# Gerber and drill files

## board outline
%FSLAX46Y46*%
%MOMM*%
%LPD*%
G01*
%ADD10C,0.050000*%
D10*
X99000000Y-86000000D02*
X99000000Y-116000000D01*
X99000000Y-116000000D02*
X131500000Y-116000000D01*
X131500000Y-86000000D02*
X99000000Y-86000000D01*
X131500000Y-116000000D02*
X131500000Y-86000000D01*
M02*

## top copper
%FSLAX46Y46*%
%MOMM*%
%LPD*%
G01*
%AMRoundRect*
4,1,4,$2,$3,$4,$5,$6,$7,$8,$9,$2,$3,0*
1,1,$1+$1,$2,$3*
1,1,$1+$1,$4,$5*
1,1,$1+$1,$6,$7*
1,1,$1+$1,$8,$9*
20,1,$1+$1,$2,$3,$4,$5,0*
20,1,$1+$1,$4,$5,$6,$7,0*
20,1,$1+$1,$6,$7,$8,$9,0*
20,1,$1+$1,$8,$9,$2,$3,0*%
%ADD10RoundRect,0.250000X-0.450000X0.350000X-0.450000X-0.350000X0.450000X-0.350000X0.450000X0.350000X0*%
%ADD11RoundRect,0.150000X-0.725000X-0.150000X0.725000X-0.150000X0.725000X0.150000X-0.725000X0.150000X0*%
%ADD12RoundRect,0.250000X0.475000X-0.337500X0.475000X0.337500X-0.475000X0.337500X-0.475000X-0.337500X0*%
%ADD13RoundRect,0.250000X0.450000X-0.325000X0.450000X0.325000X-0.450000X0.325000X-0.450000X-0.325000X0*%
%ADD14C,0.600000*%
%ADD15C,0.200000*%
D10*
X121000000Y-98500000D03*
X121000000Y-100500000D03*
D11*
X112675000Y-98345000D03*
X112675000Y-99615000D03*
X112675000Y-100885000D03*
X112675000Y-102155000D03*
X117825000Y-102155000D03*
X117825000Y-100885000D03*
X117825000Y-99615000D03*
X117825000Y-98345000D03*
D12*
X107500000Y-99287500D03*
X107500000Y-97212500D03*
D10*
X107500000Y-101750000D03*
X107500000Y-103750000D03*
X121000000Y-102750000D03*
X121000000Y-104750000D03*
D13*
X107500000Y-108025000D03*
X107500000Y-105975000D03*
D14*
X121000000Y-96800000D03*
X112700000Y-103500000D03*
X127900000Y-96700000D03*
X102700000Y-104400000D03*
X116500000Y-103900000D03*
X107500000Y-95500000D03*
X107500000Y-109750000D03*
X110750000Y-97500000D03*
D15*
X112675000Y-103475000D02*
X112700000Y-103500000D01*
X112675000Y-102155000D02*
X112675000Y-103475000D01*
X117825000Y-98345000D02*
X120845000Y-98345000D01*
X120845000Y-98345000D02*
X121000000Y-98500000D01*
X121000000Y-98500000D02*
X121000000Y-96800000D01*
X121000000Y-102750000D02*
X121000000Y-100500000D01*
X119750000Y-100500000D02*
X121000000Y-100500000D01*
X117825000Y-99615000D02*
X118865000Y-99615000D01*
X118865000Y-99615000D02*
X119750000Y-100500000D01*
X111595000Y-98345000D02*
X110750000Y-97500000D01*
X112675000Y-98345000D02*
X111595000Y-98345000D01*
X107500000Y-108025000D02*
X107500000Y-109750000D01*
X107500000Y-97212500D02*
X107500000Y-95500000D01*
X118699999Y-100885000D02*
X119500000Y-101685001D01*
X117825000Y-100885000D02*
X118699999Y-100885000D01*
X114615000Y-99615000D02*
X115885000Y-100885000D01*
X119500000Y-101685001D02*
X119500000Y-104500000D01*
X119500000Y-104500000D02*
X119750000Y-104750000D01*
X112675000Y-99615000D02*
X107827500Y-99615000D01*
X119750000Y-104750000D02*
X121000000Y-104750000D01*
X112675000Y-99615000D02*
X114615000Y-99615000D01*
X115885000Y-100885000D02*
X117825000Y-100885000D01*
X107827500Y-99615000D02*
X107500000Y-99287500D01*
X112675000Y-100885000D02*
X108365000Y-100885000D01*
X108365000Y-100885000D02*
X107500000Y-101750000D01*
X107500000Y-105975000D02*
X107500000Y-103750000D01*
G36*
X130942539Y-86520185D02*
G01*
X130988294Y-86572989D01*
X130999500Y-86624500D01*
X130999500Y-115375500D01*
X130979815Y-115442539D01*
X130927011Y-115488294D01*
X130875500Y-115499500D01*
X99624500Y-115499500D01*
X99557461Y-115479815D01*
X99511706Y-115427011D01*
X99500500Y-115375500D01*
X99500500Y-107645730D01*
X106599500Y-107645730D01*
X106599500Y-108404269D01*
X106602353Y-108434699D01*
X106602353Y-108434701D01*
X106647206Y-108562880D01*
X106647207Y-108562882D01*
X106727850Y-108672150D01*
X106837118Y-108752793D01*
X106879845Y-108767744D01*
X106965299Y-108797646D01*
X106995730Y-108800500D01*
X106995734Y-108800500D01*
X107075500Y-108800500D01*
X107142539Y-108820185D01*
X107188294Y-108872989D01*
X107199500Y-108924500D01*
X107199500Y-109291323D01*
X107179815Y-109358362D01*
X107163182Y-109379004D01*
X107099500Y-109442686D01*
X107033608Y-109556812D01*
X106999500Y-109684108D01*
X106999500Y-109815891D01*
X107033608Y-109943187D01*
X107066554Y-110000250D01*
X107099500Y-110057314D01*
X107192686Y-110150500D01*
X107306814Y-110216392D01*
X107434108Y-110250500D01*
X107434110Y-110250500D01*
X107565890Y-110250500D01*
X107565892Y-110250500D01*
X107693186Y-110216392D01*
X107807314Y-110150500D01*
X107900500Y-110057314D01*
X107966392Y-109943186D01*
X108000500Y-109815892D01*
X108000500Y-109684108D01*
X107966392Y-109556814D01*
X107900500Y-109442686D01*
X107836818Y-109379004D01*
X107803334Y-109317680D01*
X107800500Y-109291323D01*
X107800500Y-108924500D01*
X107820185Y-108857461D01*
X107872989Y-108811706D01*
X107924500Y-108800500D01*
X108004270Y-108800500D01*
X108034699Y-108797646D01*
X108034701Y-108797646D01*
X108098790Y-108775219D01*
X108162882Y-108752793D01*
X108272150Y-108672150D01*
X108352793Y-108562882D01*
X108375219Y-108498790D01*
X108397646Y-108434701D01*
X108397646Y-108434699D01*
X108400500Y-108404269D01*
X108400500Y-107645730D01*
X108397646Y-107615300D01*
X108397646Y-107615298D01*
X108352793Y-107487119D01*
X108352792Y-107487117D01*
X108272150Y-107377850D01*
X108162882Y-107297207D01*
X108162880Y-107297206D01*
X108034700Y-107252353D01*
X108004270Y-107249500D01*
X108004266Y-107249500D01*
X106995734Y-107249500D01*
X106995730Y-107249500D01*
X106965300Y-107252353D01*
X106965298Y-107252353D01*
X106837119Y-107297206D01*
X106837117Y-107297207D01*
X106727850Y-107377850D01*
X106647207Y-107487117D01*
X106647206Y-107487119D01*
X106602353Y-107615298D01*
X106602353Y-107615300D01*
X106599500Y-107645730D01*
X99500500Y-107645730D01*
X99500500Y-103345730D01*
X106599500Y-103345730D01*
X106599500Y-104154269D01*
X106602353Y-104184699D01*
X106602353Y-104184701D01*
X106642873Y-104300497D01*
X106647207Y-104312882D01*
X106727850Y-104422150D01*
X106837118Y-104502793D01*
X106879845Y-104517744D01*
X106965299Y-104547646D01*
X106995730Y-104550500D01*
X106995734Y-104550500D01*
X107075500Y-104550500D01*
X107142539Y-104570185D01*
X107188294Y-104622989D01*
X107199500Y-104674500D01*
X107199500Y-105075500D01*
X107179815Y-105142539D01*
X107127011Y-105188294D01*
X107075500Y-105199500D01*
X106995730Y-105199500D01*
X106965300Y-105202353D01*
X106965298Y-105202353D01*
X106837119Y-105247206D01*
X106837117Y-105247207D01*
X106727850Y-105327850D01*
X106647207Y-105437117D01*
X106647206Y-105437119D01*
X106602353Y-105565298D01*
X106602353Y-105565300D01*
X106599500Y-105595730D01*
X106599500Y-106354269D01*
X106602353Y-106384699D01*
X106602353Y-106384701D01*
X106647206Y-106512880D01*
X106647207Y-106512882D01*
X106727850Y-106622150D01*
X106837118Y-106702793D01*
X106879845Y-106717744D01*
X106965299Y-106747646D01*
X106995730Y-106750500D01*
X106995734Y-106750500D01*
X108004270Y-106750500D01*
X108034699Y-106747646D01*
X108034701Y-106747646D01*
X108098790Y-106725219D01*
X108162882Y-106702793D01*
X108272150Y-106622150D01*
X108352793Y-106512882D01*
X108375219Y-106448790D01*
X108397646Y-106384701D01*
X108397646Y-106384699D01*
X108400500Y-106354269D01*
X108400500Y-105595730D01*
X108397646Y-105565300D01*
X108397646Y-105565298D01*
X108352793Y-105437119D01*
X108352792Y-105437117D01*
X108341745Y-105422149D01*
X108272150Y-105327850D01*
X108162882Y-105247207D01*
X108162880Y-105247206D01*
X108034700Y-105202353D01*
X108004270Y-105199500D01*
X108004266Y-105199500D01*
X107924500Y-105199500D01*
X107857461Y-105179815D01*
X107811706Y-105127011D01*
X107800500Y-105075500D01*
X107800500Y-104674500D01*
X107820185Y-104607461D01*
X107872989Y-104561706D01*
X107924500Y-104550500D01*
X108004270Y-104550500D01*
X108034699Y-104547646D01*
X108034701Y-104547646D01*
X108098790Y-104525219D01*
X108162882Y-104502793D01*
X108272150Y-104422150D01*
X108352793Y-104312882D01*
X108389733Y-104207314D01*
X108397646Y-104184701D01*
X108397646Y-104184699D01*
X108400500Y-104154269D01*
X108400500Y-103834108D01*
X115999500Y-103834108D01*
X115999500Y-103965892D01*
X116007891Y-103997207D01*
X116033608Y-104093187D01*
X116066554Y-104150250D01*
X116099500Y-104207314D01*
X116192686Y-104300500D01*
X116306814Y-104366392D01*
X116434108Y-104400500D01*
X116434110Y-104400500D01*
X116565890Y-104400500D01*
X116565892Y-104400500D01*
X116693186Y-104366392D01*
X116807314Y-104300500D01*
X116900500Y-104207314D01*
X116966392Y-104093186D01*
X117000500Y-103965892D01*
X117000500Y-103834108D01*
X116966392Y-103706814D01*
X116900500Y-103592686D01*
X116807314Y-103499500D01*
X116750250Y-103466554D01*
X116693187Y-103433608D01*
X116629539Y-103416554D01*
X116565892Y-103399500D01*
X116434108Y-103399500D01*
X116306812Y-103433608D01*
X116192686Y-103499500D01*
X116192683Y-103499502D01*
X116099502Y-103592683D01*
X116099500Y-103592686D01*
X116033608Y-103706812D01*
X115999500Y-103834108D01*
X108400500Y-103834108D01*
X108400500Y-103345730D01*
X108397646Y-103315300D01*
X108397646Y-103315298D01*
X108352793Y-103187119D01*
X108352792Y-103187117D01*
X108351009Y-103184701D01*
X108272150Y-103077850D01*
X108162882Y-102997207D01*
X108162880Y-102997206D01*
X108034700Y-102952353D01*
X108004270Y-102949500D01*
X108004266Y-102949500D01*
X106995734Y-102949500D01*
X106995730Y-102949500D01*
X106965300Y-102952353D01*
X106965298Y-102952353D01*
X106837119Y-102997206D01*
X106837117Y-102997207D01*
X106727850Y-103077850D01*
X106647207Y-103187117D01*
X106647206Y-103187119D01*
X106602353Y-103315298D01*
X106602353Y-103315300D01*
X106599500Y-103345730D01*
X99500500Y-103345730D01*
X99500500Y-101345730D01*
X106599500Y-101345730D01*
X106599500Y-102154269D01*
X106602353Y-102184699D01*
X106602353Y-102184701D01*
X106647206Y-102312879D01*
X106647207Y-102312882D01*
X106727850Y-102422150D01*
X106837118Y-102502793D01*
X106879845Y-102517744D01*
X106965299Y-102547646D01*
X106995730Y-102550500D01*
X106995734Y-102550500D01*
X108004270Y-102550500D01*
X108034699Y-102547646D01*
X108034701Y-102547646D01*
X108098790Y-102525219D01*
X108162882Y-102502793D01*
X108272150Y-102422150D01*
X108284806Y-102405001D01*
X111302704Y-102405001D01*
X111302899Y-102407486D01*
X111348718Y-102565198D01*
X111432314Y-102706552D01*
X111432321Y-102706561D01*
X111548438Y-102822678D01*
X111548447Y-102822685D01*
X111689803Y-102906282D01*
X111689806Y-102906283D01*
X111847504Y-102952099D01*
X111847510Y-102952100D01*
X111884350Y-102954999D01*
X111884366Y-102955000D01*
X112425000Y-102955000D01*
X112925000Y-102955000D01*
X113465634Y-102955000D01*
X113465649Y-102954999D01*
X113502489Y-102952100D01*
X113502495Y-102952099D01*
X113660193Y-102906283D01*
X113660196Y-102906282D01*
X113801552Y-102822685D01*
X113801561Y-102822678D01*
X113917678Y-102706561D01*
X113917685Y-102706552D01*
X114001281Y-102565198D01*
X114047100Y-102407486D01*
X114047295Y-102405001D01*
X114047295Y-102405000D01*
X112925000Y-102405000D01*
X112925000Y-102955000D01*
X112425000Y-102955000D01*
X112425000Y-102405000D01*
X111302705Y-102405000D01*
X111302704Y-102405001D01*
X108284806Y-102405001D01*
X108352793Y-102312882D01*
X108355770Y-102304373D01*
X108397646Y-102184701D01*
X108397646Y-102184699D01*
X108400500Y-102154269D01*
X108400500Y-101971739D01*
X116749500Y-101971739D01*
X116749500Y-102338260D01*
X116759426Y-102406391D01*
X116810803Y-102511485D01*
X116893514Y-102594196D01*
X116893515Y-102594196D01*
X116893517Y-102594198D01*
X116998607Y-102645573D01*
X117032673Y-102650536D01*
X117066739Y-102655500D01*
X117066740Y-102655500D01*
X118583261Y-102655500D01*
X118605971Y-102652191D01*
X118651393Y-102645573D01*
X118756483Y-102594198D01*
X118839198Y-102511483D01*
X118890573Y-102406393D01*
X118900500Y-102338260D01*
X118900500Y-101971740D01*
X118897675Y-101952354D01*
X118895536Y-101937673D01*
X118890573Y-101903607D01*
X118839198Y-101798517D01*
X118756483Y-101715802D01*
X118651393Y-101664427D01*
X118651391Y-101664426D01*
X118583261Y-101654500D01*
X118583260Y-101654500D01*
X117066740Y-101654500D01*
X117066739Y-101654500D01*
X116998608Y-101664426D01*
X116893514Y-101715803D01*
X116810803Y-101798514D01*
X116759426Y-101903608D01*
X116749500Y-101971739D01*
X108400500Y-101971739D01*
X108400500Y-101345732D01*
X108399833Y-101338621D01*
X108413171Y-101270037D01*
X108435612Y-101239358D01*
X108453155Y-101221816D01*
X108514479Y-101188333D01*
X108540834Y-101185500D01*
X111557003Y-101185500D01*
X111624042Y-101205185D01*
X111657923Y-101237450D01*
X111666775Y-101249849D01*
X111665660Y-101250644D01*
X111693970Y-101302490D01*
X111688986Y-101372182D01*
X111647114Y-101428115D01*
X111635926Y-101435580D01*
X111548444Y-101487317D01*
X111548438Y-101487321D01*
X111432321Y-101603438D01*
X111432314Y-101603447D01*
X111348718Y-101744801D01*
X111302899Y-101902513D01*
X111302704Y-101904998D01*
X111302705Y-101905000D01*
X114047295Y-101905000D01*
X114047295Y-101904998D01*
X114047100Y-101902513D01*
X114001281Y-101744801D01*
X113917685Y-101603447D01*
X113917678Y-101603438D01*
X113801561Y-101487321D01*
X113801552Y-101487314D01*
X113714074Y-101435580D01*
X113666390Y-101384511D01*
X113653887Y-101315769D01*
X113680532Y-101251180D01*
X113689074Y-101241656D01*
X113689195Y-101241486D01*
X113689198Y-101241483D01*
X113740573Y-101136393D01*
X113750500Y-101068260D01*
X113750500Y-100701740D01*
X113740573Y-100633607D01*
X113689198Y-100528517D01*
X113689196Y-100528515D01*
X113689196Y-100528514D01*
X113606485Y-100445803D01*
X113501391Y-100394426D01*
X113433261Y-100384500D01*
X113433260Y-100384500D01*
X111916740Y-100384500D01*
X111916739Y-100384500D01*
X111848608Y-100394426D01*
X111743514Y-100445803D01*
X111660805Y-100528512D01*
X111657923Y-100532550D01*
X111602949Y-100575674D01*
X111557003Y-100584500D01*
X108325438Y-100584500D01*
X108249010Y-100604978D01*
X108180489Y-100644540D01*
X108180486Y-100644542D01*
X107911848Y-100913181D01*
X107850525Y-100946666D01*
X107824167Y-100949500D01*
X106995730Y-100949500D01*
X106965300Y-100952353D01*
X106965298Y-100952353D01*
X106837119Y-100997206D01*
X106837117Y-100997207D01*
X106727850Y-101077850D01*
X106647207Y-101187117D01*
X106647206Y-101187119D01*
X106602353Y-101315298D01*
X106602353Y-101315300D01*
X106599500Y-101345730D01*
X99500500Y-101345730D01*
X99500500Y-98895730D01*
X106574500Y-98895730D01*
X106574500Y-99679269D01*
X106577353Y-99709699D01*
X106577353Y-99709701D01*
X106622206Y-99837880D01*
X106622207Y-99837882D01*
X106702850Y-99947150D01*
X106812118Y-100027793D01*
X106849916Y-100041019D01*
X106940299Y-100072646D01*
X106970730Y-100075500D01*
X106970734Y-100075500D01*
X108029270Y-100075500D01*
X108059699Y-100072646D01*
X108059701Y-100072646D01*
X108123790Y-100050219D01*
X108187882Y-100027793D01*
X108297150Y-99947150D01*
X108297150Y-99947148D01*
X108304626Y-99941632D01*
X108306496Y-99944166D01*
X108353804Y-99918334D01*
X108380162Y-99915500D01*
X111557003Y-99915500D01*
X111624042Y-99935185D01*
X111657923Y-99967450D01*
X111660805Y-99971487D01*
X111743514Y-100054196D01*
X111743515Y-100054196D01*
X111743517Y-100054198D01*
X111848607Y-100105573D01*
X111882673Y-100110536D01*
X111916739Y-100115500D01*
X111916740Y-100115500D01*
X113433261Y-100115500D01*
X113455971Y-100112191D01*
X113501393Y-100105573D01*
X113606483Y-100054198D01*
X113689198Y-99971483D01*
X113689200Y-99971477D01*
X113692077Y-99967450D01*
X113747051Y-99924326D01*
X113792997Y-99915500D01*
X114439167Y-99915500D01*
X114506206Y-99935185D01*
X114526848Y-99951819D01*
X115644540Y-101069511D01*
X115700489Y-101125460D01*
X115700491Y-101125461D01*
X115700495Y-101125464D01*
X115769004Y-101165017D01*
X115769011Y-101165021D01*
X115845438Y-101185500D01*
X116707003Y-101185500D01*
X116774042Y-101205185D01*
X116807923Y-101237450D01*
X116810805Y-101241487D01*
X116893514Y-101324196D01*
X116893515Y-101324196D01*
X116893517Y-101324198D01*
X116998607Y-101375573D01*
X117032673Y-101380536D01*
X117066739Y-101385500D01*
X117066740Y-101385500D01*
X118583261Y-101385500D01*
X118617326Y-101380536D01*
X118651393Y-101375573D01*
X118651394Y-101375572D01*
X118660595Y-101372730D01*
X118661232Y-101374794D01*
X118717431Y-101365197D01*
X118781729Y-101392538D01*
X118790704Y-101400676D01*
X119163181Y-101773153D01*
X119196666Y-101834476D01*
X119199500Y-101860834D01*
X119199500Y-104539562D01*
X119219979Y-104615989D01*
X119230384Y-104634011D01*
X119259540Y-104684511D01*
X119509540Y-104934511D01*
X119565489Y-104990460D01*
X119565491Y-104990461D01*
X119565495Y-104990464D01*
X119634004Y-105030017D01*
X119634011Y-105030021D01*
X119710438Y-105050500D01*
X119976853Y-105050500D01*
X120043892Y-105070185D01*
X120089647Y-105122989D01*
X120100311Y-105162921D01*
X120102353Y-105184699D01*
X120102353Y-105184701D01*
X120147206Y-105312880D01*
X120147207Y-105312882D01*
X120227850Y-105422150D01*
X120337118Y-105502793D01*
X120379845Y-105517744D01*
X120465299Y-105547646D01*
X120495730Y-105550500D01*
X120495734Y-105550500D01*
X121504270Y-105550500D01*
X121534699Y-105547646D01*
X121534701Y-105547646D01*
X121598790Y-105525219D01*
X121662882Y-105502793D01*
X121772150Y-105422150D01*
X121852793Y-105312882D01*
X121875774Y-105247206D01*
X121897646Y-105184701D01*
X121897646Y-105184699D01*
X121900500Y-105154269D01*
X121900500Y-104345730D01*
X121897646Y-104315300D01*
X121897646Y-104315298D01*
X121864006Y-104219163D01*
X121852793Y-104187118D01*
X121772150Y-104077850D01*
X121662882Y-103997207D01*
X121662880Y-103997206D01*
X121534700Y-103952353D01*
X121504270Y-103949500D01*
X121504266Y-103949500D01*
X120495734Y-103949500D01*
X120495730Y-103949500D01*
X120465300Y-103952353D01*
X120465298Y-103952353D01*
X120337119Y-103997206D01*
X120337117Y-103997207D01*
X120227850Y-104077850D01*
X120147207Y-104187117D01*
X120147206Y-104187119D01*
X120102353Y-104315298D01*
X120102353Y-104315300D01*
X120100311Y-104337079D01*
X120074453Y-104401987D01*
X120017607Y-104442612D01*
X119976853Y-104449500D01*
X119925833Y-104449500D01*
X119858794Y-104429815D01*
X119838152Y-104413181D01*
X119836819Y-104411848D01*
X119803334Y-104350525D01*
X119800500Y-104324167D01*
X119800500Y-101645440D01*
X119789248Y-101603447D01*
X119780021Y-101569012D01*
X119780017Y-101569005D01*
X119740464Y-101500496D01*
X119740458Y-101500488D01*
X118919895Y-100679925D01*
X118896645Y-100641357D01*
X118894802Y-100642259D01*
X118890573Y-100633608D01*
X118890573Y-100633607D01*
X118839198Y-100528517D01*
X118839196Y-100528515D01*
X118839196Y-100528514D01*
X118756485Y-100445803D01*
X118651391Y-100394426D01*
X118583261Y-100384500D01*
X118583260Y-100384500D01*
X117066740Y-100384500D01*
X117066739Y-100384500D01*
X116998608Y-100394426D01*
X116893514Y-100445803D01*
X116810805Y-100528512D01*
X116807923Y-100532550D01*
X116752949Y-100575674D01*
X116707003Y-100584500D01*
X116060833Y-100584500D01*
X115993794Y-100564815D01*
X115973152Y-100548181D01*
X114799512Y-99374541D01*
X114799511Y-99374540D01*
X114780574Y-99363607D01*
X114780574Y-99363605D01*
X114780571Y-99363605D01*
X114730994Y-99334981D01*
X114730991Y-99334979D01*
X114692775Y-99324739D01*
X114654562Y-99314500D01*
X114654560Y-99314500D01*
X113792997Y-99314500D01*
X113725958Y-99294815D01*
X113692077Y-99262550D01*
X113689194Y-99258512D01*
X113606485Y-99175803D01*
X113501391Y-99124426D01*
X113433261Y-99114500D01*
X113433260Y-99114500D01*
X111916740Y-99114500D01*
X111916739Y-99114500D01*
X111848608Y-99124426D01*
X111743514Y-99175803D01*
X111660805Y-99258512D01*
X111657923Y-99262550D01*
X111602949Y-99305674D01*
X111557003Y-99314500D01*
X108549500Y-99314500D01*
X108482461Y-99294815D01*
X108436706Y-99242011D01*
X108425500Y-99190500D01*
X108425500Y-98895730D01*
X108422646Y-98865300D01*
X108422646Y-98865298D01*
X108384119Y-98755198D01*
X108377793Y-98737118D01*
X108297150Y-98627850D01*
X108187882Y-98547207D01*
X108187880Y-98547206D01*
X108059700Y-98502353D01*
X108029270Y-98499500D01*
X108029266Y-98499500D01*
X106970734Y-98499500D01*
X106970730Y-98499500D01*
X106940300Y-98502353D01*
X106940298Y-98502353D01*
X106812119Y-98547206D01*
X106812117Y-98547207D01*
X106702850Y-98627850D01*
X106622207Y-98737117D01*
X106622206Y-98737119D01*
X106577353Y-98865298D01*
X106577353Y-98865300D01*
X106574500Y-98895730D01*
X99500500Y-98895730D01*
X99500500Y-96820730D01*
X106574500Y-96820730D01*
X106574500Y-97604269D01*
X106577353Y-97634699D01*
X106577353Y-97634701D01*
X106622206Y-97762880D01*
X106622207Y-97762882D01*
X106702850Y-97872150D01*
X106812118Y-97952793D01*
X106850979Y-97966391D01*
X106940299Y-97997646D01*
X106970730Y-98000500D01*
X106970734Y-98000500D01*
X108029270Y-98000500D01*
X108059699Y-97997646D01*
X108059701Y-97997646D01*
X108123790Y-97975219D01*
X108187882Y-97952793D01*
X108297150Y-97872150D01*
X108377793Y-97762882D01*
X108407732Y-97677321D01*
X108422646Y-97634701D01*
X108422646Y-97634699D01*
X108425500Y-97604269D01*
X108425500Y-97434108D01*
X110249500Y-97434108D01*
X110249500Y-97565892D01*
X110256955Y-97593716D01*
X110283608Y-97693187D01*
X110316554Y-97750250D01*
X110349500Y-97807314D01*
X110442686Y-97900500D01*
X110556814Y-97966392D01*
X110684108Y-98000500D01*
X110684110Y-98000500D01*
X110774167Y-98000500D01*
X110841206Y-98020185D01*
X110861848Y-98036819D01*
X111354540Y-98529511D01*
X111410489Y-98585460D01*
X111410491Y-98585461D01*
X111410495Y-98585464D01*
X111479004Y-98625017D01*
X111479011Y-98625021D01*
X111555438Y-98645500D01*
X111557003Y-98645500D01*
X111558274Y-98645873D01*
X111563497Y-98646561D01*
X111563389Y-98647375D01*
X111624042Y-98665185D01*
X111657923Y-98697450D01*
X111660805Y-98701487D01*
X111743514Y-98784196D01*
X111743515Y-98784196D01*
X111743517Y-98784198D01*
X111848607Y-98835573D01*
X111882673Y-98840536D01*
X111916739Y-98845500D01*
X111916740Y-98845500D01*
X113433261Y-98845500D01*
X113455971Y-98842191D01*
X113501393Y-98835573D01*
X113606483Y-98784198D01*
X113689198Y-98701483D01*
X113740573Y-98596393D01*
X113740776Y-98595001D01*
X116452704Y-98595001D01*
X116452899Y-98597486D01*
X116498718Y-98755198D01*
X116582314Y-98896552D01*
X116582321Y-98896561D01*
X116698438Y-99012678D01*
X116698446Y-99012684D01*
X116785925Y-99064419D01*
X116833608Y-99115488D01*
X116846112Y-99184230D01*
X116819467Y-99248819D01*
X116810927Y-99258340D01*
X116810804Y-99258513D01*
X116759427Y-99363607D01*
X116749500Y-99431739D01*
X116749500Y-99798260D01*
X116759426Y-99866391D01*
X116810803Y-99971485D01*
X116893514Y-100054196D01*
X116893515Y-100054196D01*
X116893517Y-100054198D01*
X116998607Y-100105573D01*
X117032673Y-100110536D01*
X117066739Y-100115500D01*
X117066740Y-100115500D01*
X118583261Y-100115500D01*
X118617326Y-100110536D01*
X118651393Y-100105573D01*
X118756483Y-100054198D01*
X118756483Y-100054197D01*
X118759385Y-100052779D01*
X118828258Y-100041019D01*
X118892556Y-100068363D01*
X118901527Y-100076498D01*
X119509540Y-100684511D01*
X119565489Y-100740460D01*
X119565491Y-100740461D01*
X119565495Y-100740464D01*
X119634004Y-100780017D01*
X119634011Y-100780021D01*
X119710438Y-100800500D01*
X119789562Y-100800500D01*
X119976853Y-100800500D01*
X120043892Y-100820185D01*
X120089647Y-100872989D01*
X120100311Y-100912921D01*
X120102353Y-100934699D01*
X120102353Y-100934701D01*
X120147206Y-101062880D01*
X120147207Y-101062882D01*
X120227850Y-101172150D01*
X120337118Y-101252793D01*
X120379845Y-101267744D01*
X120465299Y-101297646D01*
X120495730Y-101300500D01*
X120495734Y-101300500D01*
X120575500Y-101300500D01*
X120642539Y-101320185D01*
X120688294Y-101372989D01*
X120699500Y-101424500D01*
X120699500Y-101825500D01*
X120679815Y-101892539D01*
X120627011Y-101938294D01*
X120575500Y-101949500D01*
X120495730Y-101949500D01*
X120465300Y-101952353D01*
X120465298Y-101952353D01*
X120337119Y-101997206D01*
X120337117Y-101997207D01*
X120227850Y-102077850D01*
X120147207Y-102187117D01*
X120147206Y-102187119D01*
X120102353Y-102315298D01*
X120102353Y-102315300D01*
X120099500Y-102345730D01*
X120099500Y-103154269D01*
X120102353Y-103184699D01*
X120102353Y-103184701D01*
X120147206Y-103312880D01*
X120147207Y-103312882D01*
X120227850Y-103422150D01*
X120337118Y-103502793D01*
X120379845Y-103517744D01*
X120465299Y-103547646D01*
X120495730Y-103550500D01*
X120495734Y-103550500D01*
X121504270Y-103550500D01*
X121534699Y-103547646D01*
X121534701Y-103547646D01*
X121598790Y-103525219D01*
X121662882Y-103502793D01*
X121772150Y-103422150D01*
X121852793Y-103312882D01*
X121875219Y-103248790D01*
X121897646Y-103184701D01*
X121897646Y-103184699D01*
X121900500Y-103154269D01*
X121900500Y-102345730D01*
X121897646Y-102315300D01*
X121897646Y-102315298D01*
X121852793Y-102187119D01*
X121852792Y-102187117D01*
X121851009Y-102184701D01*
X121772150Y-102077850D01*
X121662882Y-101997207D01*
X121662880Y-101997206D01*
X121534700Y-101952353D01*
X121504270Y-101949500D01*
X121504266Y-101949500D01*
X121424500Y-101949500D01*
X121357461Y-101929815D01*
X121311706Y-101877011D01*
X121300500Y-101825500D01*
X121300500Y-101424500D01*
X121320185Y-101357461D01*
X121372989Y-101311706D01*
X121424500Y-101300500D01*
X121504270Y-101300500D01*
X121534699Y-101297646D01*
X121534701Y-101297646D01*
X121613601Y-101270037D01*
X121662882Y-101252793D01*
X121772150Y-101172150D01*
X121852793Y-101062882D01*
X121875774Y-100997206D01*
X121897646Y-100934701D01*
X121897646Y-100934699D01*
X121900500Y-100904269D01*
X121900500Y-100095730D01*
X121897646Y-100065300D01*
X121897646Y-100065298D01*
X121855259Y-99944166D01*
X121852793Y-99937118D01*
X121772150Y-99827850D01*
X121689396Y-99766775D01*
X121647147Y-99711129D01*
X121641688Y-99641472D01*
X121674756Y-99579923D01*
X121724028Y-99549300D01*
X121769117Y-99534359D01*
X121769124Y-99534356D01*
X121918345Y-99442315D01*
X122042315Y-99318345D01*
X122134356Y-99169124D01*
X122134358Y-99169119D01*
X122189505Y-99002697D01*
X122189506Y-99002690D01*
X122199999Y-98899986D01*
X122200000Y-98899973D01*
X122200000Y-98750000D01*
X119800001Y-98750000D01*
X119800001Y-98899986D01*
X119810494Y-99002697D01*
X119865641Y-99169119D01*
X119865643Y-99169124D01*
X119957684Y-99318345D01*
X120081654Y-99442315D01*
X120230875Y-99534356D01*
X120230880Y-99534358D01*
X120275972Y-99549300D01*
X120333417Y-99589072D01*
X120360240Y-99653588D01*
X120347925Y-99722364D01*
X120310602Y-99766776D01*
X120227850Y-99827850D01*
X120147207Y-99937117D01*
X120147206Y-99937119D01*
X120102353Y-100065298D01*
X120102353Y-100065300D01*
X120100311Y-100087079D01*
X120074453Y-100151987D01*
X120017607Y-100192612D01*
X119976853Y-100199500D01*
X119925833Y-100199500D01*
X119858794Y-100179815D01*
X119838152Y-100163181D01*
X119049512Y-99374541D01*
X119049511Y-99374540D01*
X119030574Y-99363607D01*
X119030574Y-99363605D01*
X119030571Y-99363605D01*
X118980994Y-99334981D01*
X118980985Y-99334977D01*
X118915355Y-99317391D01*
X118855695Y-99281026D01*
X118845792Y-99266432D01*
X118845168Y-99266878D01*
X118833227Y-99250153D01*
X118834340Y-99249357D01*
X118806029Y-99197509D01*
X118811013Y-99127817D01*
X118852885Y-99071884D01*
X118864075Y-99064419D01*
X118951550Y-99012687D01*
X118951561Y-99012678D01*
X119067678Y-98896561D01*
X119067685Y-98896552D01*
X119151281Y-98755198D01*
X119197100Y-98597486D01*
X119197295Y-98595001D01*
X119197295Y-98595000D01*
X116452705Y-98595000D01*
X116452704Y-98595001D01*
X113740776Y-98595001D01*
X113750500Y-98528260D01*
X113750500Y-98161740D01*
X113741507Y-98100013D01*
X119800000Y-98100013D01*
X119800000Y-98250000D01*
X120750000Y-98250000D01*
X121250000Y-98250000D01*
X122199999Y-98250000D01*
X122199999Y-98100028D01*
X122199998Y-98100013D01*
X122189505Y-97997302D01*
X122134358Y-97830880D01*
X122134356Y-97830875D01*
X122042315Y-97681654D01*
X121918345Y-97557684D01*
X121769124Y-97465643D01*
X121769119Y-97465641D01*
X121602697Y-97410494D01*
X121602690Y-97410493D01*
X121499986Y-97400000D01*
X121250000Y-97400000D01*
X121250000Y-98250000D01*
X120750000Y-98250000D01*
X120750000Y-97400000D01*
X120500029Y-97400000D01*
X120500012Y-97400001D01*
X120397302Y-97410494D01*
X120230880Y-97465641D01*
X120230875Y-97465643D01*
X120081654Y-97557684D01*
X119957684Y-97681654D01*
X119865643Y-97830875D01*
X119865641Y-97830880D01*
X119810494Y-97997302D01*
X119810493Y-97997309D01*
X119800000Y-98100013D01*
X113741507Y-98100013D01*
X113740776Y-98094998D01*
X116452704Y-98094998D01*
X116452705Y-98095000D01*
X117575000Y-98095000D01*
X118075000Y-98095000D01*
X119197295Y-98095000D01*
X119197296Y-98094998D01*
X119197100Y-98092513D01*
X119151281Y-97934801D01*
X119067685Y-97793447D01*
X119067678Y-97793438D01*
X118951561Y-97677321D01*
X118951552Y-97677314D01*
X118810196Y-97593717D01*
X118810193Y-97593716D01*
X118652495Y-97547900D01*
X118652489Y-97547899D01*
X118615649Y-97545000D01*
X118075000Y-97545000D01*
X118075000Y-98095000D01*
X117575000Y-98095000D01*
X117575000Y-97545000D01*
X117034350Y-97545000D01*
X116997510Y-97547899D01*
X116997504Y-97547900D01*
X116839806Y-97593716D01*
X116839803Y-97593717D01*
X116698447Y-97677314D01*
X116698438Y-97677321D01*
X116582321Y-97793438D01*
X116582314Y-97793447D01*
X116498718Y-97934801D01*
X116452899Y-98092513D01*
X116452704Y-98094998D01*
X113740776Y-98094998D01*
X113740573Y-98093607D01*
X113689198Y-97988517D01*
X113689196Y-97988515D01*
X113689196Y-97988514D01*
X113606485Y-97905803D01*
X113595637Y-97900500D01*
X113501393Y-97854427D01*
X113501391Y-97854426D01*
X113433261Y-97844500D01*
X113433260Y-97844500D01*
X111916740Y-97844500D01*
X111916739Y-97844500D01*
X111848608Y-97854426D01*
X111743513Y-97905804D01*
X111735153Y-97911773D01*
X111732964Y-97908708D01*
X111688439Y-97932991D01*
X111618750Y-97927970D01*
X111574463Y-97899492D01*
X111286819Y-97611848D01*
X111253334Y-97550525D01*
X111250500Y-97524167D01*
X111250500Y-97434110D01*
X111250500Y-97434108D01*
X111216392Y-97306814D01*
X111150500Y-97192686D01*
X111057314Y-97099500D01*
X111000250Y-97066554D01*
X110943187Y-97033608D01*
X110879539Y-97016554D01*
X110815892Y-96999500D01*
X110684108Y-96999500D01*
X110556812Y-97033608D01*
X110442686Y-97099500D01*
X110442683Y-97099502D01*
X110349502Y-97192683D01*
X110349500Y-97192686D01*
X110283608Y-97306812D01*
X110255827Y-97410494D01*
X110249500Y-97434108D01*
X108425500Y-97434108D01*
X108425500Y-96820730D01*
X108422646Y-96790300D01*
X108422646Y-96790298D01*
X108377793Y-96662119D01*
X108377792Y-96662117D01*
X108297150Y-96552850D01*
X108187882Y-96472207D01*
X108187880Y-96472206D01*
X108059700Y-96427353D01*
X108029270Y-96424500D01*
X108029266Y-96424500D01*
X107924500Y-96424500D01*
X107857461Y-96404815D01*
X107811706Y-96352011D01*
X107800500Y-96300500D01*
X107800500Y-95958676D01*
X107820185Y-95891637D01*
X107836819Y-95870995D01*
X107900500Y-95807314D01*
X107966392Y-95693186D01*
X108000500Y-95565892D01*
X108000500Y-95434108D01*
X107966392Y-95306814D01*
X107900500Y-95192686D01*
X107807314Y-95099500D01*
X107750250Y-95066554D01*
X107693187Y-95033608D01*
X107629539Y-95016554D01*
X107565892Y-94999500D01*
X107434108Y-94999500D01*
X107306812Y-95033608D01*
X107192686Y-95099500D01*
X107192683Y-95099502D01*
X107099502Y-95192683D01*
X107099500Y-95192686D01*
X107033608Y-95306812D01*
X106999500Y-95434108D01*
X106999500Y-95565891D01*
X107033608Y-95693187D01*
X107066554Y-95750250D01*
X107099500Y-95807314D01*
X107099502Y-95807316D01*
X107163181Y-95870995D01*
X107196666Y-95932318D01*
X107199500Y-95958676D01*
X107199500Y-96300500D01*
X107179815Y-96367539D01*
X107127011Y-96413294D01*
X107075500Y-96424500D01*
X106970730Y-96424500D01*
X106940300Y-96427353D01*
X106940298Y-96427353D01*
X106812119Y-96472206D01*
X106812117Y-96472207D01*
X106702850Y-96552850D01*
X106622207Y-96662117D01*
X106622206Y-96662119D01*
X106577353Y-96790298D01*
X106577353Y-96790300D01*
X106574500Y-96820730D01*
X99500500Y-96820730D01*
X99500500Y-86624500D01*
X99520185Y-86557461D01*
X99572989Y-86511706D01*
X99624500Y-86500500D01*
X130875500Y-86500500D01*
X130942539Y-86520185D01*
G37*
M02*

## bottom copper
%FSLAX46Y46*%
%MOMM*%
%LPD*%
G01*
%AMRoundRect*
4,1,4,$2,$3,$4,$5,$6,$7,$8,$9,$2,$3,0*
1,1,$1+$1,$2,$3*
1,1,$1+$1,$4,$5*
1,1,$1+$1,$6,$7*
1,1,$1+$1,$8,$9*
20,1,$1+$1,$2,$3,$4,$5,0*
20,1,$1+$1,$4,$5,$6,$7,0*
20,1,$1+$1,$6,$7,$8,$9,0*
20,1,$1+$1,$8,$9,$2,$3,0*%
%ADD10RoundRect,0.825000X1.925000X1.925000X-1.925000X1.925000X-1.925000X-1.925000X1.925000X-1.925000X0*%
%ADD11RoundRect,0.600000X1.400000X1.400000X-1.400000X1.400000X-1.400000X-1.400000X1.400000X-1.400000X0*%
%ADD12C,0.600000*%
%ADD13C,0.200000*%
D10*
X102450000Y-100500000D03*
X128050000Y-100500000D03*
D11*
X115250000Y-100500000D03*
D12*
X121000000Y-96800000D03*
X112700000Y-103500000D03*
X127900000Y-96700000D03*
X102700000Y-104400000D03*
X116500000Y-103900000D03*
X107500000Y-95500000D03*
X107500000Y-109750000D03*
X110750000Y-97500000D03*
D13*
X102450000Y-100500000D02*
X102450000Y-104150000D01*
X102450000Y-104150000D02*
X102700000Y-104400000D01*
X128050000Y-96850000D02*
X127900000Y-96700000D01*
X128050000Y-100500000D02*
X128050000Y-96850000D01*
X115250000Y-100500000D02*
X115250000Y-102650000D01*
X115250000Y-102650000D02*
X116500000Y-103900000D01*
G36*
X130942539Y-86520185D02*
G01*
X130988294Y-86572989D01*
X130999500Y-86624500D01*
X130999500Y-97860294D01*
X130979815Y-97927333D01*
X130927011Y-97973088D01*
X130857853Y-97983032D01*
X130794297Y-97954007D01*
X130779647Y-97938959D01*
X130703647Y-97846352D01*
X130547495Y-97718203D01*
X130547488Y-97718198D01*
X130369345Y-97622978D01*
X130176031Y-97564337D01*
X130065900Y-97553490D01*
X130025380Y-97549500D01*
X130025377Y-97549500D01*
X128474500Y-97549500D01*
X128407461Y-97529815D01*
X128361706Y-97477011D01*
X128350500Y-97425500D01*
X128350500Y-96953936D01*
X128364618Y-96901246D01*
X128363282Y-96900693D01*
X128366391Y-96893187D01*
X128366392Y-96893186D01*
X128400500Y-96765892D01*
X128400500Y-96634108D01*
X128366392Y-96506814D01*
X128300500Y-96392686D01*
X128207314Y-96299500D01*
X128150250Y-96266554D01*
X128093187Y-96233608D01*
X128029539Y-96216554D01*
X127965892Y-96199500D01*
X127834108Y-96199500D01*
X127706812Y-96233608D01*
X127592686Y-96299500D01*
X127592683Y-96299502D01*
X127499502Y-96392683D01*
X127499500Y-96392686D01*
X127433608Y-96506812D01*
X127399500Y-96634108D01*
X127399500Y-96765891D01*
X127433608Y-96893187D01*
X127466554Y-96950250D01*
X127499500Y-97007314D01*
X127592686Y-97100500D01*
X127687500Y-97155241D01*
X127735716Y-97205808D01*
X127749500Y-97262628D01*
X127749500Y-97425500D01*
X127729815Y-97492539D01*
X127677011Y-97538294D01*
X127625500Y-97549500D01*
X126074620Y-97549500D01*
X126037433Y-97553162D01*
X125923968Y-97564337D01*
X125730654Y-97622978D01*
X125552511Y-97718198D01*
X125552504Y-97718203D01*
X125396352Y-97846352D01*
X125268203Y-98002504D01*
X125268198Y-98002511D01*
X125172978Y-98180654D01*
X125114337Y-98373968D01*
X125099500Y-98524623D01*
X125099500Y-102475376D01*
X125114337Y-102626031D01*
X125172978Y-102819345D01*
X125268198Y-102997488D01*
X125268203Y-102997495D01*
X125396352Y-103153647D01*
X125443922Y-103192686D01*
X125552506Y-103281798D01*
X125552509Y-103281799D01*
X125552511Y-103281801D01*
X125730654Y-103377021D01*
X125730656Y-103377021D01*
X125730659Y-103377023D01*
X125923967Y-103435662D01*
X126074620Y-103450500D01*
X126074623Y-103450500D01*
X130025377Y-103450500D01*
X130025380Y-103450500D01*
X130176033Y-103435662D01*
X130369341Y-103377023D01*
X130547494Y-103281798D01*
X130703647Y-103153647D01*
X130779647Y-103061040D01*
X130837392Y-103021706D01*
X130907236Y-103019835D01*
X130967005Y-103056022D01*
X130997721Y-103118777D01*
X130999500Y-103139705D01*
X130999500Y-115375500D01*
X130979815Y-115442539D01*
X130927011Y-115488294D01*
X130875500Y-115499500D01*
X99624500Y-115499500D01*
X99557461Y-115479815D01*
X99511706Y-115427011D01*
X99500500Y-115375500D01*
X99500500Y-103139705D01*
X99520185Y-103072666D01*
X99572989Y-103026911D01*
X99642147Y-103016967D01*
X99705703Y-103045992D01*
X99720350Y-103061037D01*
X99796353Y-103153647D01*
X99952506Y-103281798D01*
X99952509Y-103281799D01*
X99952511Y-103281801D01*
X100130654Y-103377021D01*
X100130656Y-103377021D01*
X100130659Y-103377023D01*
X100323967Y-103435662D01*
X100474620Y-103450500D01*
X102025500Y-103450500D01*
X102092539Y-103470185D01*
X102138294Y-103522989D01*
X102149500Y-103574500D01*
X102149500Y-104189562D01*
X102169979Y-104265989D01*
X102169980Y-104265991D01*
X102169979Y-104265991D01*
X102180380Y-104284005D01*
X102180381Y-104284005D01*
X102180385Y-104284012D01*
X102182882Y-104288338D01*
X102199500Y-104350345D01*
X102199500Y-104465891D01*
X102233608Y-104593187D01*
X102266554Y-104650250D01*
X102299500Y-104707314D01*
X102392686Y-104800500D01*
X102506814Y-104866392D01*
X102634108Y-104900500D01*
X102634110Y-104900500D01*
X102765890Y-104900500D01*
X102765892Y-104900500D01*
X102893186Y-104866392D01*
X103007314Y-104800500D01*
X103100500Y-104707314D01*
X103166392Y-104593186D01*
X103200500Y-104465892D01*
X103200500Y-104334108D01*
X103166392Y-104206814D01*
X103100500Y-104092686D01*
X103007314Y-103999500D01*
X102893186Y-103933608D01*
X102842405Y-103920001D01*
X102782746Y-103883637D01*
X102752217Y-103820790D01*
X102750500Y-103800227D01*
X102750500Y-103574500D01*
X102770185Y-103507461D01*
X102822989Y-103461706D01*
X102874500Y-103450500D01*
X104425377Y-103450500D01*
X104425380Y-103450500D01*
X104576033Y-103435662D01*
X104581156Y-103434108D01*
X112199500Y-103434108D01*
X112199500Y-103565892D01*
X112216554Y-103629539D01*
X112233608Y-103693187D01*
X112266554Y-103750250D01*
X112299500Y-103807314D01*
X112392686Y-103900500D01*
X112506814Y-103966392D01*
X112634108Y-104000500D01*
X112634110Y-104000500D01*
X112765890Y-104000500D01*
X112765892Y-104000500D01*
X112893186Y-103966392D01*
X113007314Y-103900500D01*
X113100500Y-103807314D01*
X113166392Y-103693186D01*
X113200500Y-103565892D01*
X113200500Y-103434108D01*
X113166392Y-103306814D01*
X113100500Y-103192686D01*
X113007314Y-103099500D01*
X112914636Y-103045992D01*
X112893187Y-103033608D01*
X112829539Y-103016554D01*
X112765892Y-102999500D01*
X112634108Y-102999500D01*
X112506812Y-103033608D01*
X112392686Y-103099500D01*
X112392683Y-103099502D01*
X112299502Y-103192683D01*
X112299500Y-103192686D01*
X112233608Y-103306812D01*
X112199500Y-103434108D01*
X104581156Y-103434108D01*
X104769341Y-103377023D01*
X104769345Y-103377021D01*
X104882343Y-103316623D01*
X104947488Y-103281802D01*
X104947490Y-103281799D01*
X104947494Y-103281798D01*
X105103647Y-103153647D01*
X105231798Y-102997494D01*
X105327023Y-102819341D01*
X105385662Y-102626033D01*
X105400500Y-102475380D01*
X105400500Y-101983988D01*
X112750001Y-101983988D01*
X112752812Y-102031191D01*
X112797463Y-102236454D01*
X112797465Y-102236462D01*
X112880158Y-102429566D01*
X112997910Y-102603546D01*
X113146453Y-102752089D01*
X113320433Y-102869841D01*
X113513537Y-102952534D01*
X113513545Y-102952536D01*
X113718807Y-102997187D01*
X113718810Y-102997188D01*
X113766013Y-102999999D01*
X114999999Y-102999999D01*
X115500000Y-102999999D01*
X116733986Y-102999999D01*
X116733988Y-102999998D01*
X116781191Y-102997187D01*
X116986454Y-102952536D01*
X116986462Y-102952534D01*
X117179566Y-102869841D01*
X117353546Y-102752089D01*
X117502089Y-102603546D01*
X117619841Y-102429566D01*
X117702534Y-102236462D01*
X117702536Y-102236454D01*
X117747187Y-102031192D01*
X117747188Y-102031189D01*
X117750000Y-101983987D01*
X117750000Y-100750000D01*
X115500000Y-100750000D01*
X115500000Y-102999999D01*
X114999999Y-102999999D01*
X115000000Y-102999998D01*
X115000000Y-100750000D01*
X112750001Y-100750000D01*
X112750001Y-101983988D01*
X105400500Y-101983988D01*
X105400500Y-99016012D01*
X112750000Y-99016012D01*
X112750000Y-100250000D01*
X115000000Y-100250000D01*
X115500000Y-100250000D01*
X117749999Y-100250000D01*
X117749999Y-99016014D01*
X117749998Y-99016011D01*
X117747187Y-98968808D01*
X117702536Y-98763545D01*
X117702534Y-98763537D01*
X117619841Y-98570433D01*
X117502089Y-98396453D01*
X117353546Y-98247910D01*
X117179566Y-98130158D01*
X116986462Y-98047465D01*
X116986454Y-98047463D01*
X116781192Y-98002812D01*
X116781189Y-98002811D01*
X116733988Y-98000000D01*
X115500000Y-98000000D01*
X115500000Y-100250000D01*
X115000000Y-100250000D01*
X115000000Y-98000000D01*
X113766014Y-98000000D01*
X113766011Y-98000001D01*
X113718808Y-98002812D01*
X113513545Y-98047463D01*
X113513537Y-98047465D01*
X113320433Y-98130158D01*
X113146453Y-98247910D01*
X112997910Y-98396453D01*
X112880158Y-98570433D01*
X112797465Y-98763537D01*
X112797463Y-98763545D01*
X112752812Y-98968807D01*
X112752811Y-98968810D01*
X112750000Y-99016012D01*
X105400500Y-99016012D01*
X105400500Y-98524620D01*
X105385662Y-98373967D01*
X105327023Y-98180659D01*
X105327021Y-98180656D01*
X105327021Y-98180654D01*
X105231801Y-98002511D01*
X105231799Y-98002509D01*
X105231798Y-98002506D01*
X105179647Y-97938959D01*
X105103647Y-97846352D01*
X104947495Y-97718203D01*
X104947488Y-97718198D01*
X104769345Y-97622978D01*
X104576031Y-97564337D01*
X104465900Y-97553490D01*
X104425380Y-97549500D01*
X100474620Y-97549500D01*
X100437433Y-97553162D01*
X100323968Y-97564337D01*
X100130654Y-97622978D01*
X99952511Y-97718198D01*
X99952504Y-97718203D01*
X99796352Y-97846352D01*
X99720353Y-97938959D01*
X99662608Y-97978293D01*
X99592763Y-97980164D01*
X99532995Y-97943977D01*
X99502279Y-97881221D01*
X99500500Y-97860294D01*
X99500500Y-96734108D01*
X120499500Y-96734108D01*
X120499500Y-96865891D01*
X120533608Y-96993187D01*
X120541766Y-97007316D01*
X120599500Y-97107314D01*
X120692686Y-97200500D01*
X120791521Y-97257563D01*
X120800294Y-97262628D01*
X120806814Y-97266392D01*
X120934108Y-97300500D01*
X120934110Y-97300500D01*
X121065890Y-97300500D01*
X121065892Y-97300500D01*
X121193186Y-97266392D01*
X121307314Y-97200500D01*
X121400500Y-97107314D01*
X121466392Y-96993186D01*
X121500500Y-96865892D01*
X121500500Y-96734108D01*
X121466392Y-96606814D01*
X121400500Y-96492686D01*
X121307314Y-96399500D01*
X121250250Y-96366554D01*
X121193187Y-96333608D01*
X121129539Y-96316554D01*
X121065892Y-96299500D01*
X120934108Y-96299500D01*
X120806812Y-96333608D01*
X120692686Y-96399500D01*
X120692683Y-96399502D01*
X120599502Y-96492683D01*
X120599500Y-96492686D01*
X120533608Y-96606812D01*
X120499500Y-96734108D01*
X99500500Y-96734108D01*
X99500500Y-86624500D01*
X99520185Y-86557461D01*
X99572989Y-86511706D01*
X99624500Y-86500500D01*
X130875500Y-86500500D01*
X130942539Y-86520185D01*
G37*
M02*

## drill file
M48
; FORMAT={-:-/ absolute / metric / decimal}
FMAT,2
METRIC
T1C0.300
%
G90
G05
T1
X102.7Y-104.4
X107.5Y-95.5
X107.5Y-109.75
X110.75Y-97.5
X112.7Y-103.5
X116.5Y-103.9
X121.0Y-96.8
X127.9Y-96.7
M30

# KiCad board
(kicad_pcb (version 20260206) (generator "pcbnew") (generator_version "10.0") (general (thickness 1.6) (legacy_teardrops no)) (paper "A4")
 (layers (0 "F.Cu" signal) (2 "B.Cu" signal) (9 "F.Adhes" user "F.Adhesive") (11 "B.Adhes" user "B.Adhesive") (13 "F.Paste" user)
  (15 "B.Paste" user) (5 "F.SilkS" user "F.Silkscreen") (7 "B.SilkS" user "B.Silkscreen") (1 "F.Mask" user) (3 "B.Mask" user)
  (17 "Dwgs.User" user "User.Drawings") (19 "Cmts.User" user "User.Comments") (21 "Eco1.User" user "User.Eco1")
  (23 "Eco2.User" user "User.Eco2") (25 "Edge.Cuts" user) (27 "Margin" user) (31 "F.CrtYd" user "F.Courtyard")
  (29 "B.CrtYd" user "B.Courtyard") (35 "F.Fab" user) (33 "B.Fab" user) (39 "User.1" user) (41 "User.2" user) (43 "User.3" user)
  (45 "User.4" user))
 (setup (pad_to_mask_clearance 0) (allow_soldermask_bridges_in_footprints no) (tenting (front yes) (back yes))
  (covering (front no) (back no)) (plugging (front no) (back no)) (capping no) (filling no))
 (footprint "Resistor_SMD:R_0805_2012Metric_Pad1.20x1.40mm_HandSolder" (layer "F.Cu") (at 121 99.5 -90)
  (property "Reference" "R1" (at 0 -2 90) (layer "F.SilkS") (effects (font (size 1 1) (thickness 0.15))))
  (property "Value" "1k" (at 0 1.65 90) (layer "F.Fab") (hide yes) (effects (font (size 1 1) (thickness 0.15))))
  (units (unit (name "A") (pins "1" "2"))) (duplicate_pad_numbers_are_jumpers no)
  (pad "1" smd roundrect (at -1 0 270) (size 1.2 1.4) (layers "F.Cu" "F.Mask" "F.Paste") (roundrect_rratio 0.208333) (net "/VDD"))
  (pad "2" smd roundrect (at 1 0 270) (size 1.2 1.4) (layers "F.Cu" "F.Mask" "F.Paste") (roundrect_rratio 0.208333) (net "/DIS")))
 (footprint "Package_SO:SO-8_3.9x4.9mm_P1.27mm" (layer "F.Cu") (at 115.25 100.25)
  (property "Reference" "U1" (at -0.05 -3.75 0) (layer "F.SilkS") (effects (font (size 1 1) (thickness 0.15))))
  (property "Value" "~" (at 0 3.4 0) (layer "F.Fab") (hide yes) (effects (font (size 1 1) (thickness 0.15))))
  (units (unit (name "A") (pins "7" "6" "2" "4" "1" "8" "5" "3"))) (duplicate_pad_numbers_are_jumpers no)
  (pad "1" smd roundrect (at -2.575 -1.905) (size 1.75 0.6) (layers "F.Cu" "F.Mask" "F.Paste") (roundrect_rratio 0.25) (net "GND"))
  (pad "2" smd roundrect (at -2.575 -0.635) (size 1.75 0.6) (layers "F.Cu" "F.Mask" "F.Paste") (roundrect_rratio 0.25) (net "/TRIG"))
  (pad "3" smd roundrect (at -2.575 0.635) (size 1.75 0.6) (layers "F.Cu" "F.Mask" "F.Paste") (roundrect_rratio 0.25) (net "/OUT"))
  (pad "4" smd roundrect (at -2.575 1.905) (size 1.75 0.6) (layers "F.Cu" "F.Mask" "F.Paste") (roundrect_rratio 0.25) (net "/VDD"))
  (pad "5" smd roundrect (at 2.575 1.905) (size 1.75 0.6) (layers "F.Cu" "F.Mask" "F.Paste") (roundrect_rratio 0.25)
   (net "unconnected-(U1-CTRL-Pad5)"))
  (pad "6" smd roundrect (at 2.575 0.635) (size 1.75 0.6) (layers "F.Cu" "F.Mask" "F.Paste") (roundrect_rratio 0.25) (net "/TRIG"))
  (pad "7" smd roundrect (at 2.575 -0.635) (size 1.75 0.6) (layers "F.Cu" "F.Mask" "F.Paste") (roundrect_rratio 0.25) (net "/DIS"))
  (pad "8" smd roundrect (at 2.575 -1.905) (size 1.75 0.6) (layers "F.Cu" "F.Mask" "F.Paste") (roundrect_rratio 0.25) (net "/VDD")))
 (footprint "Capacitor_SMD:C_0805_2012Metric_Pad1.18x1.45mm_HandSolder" (layer "F.Cu") (at 107.5 98.25 90)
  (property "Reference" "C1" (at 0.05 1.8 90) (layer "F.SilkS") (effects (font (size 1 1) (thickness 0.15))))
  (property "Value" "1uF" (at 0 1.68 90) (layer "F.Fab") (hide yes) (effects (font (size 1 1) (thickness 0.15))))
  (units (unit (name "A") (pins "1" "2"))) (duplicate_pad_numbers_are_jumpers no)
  (pad "1" smd roundrect (at -1.0375 0 90) (size 1.175 1.45) (layers "F.Cu" "F.Mask" "F.Paste") (roundrect_rratio 0.212766) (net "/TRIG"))
  (pad "2" smd roundrect (at 1.0375 0 90) (size 1.175 1.45) (layers "F.Cu" "F.Mask" "F.Paste") (roundrect_rratio 0.212766) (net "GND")))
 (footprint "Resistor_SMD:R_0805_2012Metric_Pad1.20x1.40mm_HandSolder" (layer "F.Cu") (at 107.5 102.75 -90)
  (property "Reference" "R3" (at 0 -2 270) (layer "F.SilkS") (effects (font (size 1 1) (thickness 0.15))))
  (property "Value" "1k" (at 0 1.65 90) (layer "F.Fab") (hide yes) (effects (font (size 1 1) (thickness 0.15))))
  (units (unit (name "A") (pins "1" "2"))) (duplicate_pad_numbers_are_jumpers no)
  (pad "1" smd roundrect (at -1 0 270) (size 1.2 1.4) (layers "F.Cu" "F.Mask" "F.Paste") (roundrect_rratio 0.208333) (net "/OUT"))
  (pad "2" smd roundrect (at 1 0 270) (size 1.2 1.4) (layers "F.Cu" "F.Mask" "F.Paste") (roundrect_rratio 0.208333) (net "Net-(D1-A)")))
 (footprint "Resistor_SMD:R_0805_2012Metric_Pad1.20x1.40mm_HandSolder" (layer "F.Cu") (at 121 103.75 -90)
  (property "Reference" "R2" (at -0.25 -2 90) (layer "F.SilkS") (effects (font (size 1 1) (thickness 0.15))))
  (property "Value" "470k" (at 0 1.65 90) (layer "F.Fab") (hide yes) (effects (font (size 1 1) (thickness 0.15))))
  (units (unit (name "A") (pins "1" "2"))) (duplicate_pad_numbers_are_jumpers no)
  (pad "1" smd roundrect (at -1 0 270) (size 1.2 1.4) (layers "F.Cu" "F.Mask" "F.Paste") (roundrect_rratio 0.208333) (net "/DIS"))
  (pad "2" smd roundrect (at 1 0 270) (size 1.2 1.4) (layers "F.Cu" "F.Mask" "F.Paste") (roundrect_rratio 0.208333) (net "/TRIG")))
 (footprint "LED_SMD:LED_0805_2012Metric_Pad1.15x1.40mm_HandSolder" (layer "F.Cu") (at 107.5 107 90)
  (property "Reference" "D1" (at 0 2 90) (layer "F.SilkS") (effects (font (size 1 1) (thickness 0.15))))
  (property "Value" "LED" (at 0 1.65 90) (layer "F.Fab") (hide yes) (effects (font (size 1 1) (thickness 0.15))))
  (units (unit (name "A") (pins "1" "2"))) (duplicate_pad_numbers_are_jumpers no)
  (pad "1" smd roundrect (at -1.025 0 90) (size 1.15 1.4) (layers "F.Cu" "F.Mask" "F.Paste") (roundrect_rratio 0.217391) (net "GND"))
  (pad "2" smd roundrect (at 1.025 0 90) (size 1.15 1.4) (layers "F.Cu" "F.Mask" "F.Paste") (roundrect_rratio 0.217391) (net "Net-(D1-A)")))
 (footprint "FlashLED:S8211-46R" (layer "B.Cu") (at 115.25 100.55 180)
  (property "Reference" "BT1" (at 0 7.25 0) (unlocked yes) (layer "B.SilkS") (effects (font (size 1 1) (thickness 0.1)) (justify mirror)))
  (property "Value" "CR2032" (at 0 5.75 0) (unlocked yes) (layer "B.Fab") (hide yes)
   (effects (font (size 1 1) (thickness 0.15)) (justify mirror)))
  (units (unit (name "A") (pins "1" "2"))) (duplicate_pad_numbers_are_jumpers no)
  (pad "1" smd roundrect (at 12.8 0.05 180) (size 5.5 5.5) (layers "B.Cu" "B.Mask" "B.Paste") (roundrect_rratio 0.15) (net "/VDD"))
  (pad "2" smd roundrect (at -12.8 0.05 180) (size 5.5 5.5) (layers "B.Cu" "B.Mask" "B.Paste") (roundrect_rratio 0.15) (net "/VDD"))
  (pad "GND" smd roundrect (at 0 0.05 180) (size 4 4) (layers "B.Cu" "B.Mask" "B.Paste") (roundrect_rratio 0.15) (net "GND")))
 (gr_line (start 99 86) (end 99 116) (stroke (width 0.05) (type default)) (layer "Edge.Cuts"))
 (gr_line (start 99 116) (end 131.5 116) (stroke (width 0.05) (type default)) (layer "Edge.Cuts"))
 (gr_line (start 131.5 86) (end 99 86) (stroke (width 0.05) (type default)) (layer "Edge.Cuts"))
 (gr_line (start 131.5 116) (end 131.5 86) (stroke (width 0.05) (type default)) (layer "Edge.Cuts"))
 (segment (start 112.675 103.475) (end 112.7 103.5) (width 0.2) (layer "F.Cu") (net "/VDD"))
 (segment (start 112.675 102.155) (end 112.675 103.475) (width 0.2) (layer "F.Cu") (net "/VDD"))
 (segment (start 117.825 98.345) (end 120.845 98.345) (width 0.2) (layer "F.Cu") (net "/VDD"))
 (segment (start 120.845 98.345) (end 121 98.5) (width 0.2) (layer "F.Cu") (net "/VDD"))
 (segment (start 121 98.5) (end 121 96.8) (width 0.2) (layer "F.Cu") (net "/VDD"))
 (via (at 121 96.8) (size 0.6) (drill 0.3) (layers "F.Cu" "B.Cu") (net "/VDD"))
 (via (at 112.7 103.5) (size 0.6) (drill 0.3) (layers "F.Cu" "B.Cu") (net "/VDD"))
 (via (at 127.9 96.7) (size 0.6) (drill 0.3) (layers "F.Cu" "B.Cu") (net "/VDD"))
 (via (at 102.7 104.4) (size 0.6) (drill 0.3) (layers "F.Cu" "B.Cu") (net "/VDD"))
 (segment (start 102.45 100.5) (end 102.45 104.15) (width 0.2) (layer "B.Cu") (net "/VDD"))
 (segment (start 102.45 104.15) (end 102.7 104.4) (width 0.2) (layer "B.Cu") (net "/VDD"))
 (segment (start 128.05 96.85) (end 127.9 96.7) (width 0.2) (layer "B.Cu") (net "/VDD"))
 (segment (start 128.05 100.5) (end 128.05 96.85) (width 0.2) (layer "B.Cu") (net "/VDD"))
 (segment (start 121 102.75) (end 121 100.5) (width 0.2) (layer "F.Cu") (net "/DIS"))
 (segment (start 119.75 100.5) (end 121 100.5) (width 0.2) (layer "F.Cu") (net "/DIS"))
 (segment (start 117.825 99.615) (end 118.865 99.615) (width 0.2) (layer "F.Cu") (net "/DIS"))
 (segment (start 118.865 99.615) (end 119.75 100.5) (width 0.2) (layer "F.Cu") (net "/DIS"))
 (segment (start 111.595 98.345) (end 110.75 97.5) (width 0.2) (layer "F.Cu") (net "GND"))
 (segment (start 112.675 98.345) (end 111.595 98.345) (width 0.2) (layer "F.Cu") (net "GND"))
 (segment (start 107.5 108.025) (end 107.5 109.75) (width 0.2) (layer "F.Cu") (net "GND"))
 (segment (start 107.5 97.2125) (end 107.5 95.5) (width 0.2) (layer "F.Cu") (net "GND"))
 (via (at 116.5 103.9) (size 0.6) (drill 0.3) (layers "F.Cu" "B.Cu") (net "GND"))
 (via (at 107.5 95.5) (size 0.6) (drill 0.3) (layers "F.Cu" "B.Cu") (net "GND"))
 (via (at 107.5 109.75) (size 0.6) (drill 0.3) (layers "F.Cu" "B.Cu") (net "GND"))
 (via (at 110.75 97.5) (size 0.6) (drill 0.3) (layers "F.Cu" "B.Cu") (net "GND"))
 (segment (start 115.25 100.5) (end 115.25 102.65) (width 0.2) (layer "B.Cu") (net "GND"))
 (segment (start 115.25 102.65) (end 116.5 103.9) (width 0.2) (layer "B.Cu") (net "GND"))
 (segment (start 118.699999 100.885) (end 119.5 101.685001) (width 0.2) (layer "F.Cu") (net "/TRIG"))
 (segment (start 117.825 100.885) (end 118.699999 100.885) (width 0.2) (layer "F.Cu") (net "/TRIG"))
 (segment (start 114.615 99.615) (end 115.885 100.885) (width 0.2) (layer "F.Cu") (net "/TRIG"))
 (segment (start 119.5 101.685001) (end 119.5 104.5) (width 0.2) (layer "F.Cu") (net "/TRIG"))
 (segment (start 119.5 104.5) (end 119.75 104.75) (width 0.2) (layer "F.Cu") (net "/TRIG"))
 (segment (start 112.675 99.615) (end 107.8275 99.615) (width 0.2) (layer "F.Cu") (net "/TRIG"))
 (segment (start 119.75 104.75) (end 121 104.75) (width 0.2) (layer "F.Cu") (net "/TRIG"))
 (segment (start 112.675 99.615) (end 114.615 99.615) (width 0.2) (layer "F.Cu") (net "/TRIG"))
 (segment (start 115.885 100.885) (end 117.825 100.885) (width 0.2) (layer "F.Cu") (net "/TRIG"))
 (segment (start 107.8275 99.615) (end 107.5 99.2875) (width 0.2) (layer "F.Cu") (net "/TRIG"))
 (segment (start 112.675 100.885) (end 108.365 100.885) (width 0.2) (layer "F.Cu") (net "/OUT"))
 (segment (start 108.365 100.885) (end 107.5 101.75) (width 0.2) (layer "F.Cu") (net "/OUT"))
 (segment (start 107.5 105.975) (end 107.5 103.75) (width 0.2) (layer "F.Cu") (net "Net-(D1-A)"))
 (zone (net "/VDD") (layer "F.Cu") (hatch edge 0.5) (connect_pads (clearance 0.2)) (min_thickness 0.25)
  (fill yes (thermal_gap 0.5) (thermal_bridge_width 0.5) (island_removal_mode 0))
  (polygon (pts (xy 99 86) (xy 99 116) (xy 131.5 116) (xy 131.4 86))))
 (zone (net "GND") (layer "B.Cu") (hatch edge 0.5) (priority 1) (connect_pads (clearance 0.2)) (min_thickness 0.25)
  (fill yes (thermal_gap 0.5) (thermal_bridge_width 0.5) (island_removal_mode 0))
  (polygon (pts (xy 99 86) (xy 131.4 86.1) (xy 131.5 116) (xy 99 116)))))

